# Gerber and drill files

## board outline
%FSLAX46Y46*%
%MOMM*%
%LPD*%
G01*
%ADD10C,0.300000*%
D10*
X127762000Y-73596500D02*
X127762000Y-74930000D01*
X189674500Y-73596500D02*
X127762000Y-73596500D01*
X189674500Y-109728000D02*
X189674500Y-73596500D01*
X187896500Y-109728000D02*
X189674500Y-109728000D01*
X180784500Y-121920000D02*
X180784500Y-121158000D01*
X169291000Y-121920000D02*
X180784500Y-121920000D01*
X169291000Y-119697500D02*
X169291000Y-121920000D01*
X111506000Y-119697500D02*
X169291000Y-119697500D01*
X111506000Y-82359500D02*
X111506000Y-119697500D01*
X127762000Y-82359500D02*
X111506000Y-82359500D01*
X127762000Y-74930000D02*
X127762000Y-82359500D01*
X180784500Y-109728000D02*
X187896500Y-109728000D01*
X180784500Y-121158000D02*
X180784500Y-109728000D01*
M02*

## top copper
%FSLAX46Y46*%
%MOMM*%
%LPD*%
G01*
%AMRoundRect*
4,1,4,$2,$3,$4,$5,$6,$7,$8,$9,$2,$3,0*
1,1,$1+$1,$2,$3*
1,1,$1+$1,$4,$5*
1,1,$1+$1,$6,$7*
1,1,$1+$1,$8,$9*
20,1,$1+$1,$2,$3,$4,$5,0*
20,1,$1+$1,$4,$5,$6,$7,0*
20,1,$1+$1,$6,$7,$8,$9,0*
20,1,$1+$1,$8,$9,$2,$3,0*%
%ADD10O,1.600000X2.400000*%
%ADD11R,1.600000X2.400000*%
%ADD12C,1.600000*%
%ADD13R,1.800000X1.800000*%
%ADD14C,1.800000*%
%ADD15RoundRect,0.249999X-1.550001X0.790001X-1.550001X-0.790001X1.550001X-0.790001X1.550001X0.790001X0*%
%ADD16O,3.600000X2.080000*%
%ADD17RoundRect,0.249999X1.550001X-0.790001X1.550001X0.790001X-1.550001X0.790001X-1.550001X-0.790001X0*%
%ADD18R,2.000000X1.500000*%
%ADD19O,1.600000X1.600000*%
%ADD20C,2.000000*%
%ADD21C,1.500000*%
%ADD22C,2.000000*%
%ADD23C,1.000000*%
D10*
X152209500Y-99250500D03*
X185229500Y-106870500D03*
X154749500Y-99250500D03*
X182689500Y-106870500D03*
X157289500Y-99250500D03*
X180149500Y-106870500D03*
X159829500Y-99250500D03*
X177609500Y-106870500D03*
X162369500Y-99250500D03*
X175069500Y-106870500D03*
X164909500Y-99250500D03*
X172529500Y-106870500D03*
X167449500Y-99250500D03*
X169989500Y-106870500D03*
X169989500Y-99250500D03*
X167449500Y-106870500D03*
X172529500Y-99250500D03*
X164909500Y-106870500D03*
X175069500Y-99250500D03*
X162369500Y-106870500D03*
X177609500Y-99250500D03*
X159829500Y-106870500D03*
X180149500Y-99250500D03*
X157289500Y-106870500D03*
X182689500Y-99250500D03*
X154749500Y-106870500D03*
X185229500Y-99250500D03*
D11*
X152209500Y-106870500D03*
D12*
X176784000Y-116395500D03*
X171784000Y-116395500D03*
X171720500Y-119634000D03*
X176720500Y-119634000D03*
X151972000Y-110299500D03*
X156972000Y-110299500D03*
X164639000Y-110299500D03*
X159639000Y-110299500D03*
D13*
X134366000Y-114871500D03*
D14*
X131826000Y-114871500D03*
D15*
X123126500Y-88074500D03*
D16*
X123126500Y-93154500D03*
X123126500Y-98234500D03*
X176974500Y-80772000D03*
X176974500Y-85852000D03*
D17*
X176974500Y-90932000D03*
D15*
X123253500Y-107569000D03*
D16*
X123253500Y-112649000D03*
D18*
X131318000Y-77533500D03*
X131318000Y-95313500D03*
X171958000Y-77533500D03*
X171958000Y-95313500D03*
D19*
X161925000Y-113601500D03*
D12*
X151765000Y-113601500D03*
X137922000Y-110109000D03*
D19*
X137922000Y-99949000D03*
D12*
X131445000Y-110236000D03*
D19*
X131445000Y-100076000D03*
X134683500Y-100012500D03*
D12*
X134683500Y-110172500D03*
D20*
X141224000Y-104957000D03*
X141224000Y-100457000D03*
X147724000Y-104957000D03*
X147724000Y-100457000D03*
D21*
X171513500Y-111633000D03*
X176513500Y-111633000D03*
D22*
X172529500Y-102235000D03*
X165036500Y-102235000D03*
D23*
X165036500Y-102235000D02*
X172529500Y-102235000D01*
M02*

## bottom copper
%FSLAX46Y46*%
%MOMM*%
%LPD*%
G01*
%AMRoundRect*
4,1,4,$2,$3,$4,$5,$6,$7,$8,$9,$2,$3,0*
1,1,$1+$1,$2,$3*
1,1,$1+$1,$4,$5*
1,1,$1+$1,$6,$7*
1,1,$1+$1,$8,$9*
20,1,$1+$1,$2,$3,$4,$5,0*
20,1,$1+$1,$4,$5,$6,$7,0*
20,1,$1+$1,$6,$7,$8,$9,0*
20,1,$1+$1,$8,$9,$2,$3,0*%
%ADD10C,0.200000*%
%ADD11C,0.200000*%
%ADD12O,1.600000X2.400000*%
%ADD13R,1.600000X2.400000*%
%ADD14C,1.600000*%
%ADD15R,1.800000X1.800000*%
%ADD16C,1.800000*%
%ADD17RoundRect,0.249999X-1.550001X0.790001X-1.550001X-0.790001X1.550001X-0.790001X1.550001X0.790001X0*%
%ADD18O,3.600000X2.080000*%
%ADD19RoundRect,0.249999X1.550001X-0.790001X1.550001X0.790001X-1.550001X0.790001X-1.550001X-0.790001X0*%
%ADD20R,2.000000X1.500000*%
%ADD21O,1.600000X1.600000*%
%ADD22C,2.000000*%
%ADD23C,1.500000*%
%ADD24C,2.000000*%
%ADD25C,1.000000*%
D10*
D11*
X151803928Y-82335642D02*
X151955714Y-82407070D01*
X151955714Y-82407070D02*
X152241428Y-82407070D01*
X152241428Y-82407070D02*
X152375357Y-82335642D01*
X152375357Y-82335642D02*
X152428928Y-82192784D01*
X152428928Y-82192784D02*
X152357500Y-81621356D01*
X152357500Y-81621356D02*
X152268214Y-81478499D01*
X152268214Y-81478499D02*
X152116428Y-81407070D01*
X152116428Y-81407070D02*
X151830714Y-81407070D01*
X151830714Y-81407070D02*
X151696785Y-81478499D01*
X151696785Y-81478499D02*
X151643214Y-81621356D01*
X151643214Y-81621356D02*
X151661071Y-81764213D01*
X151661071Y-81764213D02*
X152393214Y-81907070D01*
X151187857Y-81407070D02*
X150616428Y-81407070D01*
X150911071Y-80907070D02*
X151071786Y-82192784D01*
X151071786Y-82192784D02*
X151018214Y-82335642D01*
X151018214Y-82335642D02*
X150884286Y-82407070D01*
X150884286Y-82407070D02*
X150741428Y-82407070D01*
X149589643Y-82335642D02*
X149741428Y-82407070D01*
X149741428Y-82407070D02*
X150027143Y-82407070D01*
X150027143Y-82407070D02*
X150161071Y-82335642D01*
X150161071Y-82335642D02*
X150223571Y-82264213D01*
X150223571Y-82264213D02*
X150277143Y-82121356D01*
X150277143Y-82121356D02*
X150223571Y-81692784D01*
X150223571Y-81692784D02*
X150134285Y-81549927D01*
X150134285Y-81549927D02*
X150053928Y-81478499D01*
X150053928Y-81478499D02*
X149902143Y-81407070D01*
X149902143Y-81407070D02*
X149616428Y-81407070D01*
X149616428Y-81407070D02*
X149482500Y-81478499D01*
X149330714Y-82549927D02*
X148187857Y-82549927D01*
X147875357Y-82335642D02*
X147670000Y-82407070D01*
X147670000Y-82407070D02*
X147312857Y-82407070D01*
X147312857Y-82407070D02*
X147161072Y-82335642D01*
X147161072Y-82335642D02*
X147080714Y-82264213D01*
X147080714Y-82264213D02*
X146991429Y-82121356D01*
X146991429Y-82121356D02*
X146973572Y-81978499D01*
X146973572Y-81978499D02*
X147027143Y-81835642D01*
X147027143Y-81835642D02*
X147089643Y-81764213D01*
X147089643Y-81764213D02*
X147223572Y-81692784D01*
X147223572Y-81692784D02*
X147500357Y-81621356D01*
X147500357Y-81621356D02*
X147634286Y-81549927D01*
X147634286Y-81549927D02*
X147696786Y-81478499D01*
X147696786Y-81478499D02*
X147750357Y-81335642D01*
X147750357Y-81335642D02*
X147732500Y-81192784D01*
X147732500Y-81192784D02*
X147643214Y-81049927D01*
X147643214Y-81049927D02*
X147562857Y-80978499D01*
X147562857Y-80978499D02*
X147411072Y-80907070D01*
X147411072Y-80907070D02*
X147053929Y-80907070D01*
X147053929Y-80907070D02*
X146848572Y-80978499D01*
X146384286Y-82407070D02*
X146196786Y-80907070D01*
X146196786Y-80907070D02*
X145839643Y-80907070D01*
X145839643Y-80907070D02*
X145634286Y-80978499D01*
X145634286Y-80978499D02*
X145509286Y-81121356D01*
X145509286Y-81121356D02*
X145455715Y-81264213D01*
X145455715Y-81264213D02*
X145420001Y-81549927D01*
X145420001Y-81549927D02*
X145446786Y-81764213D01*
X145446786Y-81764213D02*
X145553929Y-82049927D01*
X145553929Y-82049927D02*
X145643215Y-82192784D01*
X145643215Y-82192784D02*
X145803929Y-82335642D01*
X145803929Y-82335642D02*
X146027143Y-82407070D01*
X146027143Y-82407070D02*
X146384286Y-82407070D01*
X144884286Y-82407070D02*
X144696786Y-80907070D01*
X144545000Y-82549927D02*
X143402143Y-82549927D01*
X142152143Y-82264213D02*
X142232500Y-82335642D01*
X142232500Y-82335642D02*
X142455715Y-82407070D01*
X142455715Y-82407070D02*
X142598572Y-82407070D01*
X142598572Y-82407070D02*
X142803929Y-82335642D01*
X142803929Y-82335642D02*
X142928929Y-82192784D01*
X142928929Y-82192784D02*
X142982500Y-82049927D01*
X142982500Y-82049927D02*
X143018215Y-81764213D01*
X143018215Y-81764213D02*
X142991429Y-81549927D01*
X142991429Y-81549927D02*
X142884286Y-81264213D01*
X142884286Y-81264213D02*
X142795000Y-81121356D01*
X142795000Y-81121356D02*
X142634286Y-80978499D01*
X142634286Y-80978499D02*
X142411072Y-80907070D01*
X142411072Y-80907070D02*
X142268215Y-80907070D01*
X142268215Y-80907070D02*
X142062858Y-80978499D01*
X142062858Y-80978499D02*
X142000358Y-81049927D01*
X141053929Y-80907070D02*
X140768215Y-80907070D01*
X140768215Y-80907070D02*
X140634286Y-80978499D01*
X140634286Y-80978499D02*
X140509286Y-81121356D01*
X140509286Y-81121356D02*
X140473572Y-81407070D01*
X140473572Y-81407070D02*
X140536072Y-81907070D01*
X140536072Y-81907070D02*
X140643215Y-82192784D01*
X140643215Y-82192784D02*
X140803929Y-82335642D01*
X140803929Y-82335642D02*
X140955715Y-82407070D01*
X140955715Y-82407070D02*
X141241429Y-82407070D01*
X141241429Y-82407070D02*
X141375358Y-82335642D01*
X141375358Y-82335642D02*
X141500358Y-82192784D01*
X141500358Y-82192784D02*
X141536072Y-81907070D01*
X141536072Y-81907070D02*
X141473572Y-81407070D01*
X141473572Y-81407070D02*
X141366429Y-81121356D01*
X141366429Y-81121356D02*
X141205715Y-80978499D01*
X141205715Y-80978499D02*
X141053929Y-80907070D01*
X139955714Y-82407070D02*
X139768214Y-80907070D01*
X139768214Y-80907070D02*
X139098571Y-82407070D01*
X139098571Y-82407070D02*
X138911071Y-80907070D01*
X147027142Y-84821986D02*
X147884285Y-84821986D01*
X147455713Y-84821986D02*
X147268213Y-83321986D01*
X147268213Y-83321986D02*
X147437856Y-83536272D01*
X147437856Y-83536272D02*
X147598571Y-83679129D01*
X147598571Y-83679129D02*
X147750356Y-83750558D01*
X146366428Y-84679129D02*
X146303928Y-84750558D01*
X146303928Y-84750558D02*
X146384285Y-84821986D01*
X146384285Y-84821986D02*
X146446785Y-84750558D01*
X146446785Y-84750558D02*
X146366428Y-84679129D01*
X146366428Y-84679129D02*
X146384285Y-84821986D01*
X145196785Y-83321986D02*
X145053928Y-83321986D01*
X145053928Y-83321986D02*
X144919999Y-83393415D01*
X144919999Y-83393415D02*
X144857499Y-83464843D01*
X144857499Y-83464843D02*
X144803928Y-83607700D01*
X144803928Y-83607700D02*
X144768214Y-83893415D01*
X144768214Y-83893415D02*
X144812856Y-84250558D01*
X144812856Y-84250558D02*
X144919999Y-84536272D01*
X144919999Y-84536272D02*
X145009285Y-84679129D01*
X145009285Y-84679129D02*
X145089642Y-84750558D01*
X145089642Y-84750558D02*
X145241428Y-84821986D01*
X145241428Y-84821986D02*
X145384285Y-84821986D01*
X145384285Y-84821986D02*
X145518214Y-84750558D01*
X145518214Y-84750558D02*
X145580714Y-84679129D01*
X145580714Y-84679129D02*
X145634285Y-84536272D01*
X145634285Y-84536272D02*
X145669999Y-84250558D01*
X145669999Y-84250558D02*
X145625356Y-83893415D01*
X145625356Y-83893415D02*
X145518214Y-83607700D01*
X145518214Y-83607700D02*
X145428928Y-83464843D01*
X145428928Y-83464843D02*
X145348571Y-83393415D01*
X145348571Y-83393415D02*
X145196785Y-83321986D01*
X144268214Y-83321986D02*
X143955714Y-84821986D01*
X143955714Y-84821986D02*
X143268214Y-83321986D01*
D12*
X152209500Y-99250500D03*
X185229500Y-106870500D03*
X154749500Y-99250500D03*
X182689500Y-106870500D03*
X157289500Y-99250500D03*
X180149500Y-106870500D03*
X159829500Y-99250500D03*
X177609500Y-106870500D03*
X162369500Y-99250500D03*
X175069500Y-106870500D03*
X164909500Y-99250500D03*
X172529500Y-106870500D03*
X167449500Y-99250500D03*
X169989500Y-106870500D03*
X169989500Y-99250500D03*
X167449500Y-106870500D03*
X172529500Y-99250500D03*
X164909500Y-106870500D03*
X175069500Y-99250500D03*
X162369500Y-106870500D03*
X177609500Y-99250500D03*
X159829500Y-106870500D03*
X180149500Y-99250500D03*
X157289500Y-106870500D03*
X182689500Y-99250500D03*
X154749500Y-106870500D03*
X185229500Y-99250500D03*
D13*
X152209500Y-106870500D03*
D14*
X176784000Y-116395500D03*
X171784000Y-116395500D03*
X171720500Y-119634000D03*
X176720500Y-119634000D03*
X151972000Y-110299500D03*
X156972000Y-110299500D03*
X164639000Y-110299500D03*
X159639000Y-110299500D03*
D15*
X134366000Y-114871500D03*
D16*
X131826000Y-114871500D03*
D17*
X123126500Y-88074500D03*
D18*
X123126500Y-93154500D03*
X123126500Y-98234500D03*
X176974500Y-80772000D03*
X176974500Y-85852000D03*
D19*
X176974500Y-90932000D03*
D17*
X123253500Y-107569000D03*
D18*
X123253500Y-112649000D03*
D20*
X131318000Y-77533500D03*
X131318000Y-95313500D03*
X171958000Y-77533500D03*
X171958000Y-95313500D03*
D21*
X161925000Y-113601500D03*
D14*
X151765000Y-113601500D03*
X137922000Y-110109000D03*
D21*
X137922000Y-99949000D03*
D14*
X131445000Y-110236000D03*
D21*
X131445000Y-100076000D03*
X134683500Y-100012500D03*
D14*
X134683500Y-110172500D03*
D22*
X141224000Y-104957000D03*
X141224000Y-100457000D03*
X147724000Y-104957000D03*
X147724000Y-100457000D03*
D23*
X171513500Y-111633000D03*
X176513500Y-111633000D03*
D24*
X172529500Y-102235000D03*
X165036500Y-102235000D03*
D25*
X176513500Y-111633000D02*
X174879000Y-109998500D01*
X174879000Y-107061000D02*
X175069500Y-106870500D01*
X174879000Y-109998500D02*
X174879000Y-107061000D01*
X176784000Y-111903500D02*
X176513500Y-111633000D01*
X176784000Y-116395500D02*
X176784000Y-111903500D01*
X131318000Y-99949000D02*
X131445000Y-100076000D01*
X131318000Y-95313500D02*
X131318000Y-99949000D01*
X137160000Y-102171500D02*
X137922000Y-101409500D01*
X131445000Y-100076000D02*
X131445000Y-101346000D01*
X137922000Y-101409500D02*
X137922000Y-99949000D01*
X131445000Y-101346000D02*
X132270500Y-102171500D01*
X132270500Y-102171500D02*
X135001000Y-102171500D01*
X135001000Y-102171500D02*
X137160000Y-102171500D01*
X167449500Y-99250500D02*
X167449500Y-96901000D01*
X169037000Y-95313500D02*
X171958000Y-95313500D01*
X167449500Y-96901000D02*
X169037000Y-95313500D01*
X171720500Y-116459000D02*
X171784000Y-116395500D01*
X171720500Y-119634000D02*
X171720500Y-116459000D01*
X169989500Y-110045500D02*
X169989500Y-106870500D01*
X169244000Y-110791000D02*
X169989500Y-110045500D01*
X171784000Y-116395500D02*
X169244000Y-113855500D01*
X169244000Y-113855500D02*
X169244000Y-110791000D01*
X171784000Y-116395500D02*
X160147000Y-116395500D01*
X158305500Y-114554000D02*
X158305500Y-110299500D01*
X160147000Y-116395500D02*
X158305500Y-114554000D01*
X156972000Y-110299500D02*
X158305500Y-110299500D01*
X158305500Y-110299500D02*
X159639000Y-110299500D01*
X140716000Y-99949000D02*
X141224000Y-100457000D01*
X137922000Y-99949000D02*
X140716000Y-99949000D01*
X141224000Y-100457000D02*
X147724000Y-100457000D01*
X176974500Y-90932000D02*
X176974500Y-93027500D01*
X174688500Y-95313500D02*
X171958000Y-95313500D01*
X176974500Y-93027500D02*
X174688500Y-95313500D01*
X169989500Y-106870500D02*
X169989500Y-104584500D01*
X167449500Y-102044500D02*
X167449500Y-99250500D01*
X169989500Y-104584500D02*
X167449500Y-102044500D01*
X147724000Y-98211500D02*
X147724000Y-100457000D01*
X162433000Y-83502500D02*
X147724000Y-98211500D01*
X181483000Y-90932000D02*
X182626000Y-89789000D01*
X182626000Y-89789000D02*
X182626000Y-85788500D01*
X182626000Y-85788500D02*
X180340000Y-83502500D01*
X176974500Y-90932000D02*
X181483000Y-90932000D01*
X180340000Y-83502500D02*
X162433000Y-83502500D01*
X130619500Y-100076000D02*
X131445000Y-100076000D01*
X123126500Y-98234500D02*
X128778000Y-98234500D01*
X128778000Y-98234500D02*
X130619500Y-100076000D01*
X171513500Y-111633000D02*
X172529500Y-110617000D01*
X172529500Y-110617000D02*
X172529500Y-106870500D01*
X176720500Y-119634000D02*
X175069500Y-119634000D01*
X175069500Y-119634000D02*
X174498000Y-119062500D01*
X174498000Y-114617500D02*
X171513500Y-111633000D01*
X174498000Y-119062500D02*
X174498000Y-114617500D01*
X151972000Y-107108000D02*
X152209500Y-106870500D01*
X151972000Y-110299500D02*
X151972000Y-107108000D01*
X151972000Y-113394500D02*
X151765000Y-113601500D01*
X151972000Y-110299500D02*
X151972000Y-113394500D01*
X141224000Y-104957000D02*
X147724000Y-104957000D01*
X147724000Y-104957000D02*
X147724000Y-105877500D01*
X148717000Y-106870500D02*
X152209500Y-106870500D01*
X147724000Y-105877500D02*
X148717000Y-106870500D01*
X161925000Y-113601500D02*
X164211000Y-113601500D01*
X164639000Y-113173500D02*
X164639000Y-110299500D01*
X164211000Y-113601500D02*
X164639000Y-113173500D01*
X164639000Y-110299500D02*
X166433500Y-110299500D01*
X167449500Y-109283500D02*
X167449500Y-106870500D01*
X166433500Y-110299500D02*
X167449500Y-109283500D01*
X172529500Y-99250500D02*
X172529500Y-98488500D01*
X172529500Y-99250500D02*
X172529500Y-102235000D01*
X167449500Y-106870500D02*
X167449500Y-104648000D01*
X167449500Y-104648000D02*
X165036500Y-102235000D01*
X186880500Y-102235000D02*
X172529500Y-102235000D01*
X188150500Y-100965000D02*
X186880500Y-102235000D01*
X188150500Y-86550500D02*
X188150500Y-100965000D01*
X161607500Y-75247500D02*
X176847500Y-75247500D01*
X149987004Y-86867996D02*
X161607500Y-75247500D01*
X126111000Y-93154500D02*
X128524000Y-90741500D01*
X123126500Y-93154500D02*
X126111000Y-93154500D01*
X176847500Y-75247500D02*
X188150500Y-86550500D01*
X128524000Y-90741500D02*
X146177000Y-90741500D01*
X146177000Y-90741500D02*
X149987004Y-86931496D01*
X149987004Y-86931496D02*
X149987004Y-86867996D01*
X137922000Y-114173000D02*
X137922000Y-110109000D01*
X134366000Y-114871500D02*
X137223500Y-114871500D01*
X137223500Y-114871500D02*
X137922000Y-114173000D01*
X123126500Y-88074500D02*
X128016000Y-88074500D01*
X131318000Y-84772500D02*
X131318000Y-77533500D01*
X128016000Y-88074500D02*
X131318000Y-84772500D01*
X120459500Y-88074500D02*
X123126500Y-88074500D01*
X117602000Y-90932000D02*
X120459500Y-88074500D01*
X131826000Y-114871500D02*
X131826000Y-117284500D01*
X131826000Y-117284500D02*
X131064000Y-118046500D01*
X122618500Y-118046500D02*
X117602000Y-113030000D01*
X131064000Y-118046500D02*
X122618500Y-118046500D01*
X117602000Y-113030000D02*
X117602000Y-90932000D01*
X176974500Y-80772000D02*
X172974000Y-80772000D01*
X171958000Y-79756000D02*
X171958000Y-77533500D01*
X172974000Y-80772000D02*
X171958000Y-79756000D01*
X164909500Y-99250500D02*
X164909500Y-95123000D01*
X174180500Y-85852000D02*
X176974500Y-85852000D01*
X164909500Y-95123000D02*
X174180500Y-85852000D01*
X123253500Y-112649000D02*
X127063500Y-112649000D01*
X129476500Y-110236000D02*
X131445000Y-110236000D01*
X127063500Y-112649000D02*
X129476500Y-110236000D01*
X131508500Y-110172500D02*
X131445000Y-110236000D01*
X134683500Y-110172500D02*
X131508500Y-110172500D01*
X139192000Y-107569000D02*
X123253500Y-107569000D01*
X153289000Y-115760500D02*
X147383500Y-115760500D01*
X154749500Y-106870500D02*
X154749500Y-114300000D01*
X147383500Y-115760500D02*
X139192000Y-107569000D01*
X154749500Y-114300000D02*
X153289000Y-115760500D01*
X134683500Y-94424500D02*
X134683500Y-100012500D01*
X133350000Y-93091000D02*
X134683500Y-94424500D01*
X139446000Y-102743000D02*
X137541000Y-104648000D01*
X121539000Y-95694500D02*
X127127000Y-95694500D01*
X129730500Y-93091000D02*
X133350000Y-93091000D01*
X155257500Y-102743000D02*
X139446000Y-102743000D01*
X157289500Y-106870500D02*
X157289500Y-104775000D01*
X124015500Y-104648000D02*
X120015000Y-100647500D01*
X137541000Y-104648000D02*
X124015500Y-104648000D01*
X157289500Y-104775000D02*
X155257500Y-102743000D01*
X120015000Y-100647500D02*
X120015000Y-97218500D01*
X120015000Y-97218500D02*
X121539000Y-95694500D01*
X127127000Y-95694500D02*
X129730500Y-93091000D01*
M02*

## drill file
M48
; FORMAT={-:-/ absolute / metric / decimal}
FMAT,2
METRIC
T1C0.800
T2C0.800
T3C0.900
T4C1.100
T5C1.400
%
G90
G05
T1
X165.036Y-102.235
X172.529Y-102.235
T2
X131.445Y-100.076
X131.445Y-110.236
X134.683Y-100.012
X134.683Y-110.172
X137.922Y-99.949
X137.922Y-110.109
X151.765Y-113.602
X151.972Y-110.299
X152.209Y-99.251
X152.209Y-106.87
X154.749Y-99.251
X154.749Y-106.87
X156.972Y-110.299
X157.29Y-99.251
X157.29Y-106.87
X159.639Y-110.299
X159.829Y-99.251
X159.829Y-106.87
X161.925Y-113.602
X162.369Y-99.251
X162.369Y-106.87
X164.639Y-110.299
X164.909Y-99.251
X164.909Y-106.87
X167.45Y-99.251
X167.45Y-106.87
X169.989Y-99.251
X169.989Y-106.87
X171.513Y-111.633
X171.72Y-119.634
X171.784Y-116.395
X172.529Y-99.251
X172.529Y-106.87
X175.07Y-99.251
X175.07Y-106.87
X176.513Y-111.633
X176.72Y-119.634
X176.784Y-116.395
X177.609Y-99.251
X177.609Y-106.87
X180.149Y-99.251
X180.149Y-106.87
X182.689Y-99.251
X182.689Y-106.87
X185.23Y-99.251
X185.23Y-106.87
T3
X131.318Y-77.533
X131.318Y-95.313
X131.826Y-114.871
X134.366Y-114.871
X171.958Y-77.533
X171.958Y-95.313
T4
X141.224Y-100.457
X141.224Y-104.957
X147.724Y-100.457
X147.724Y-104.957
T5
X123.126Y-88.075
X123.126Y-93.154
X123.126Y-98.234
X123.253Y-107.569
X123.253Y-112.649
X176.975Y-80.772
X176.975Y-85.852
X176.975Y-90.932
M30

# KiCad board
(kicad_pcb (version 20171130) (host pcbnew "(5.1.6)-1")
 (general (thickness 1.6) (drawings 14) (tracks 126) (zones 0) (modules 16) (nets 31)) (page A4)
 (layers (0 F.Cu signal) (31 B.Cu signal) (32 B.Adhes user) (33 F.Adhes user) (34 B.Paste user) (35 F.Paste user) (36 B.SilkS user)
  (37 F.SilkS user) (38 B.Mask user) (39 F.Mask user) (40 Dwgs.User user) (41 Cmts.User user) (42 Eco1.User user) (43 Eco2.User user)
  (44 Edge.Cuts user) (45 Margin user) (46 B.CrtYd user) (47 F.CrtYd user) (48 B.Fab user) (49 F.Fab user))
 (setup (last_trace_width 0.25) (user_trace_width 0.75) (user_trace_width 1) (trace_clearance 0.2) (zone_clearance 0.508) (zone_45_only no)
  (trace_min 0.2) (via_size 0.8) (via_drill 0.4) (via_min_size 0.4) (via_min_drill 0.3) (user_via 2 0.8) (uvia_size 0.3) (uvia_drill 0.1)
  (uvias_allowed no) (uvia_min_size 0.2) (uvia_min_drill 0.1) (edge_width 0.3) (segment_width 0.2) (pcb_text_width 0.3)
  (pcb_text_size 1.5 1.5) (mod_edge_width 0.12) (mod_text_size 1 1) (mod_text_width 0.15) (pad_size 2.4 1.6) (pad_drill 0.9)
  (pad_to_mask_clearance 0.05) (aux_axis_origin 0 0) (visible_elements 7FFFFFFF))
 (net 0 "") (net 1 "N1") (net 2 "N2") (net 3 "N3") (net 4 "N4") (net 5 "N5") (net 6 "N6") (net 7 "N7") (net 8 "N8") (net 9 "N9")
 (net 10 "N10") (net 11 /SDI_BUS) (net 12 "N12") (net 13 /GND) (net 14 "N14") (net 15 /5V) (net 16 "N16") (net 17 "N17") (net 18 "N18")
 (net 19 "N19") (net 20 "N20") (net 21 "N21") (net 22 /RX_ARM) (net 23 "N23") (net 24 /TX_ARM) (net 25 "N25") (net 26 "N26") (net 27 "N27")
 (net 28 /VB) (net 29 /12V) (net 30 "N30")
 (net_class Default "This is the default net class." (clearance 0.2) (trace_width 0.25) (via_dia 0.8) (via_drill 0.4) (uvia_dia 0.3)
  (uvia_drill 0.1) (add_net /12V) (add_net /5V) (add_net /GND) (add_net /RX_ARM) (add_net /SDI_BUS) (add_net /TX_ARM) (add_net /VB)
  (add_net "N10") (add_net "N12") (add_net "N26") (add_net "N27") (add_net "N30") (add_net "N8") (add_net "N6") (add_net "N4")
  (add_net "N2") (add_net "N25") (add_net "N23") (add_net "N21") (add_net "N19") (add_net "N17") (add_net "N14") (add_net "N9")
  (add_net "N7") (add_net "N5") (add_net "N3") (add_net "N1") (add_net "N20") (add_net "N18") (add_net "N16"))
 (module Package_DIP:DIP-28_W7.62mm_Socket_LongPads (layer F.Cu) (at 152.2095 106.8705 90)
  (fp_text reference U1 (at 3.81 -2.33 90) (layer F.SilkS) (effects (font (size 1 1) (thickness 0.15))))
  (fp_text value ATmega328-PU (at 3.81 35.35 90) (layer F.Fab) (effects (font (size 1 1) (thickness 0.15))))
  (pad 28 thru_hole oval (at 7.62 0 90) (size 2.4 1.6) (drill 0.8) (layers *.Cu *.Mask) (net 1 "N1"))
  (pad 14 thru_hole oval (at 0 33.02 90) (size 2.4 1.6) (drill 0.8) (layers *.Cu *.Mask) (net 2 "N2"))
  (pad 27 thru_hole oval (at 7.62 2.54 90) (size 2.4 1.6) (drill 0.8) (layers *.Cu *.Mask) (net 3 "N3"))
  (pad 13 thru_hole oval (at 0 30.48 90) (size 2.4 1.6) (drill 0.8) (layers *.Cu *.Mask) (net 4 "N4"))
  (pad 26 thru_hole oval (at 7.62 5.08 90) (size 2.4 1.6) (drill 0.8) (layers *.Cu *.Mask) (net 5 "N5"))
  (pad 12 thru_hole oval (at 0 27.94 90) (size 2.4 1.6) (drill 0.8) (layers *.Cu *.Mask) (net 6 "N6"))
  (pad 25 thru_hole oval (at 7.62 7.62 90) (size 2.4 1.6) (drill 0.8) (layers *.Cu *.Mask) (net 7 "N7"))
  (pad 11 thru_hole oval (at 0 25.4 90) (size 2.4 1.6) (drill 0.8) (layers *.Cu *.Mask) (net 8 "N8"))
  (pad 24 thru_hole oval (at 7.62 10.16 90) (size 2.4 1.6) (drill 0.8) (layers *.Cu *.Mask) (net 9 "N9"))
  (pad 10 thru_hole oval (at 0 22.86 90) (size 2.4 1.6) (drill 0.8) (layers *.Cu *.Mask) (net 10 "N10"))
  (pad 23 thru_hole oval (at 7.62 12.7 90) (size 2.4 1.6) (drill 0.8) (layers *.Cu *.Mask) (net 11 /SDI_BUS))
  (pad 9 thru_hole oval (at 0 20.32 90) (size 2.4 1.6) (drill 0.8) (layers *.Cu *.Mask) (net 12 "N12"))
  (pad 22 thru_hole oval (at 7.62 15.24 90) (size 2.4 1.6) (drill 0.8) (layers *.Cu *.Mask) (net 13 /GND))
  (pad 8 thru_hole oval (at 0 17.78 90) (size 2.4 1.6) (drill 0.8) (layers *.Cu *.Mask) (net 13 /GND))
  (pad 21 thru_hole oval (at 7.62 17.78 90) (size 2.4 1.6) (drill 0.8) (layers *.Cu *.Mask) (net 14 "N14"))
  (pad 7 thru_hole oval (at 0 15.24 90) (size 2.4 1.6) (drill 0.8) (layers *.Cu *.Mask) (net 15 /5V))
  (pad 20 thru_hole oval (at 7.62 20.32 90) (size 2.4 1.6) (drill 0.8) (layers *.Cu *.Mask) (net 15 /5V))
  (pad 6 thru_hole oval (at 0 12.7 90) (size 2.4 1.6) (drill 0.8) (layers *.Cu *.Mask) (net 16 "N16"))
  (pad 19 thru_hole oval (at 7.62 22.86 90) (size 2.4 1.6) (drill 0.8) (layers *.Cu *.Mask) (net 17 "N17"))
  (pad 5 thru_hole oval (at 0 10.16 90) (size 2.4 1.6) (drill 0.8) (layers *.Cu *.Mask) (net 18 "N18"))
  (pad 18 thru_hole oval (at 7.62 25.4 90) (size 2.4 1.6) (drill 0.8) (layers *.Cu *.Mask) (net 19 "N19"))
  (pad 4 thru_hole oval (at 0 7.62 90) (size 2.4 1.6) (drill 0.8) (layers *.Cu *.Mask) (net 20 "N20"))
  (pad 17 thru_hole oval (at 7.62 27.94 90) (size 2.4 1.6) (drill 0.8) (layers *.Cu *.Mask) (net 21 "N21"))
  (pad 3 thru_hole oval (at 0 5.08 90) (size 2.4 1.6) (drill 0.8) (layers *.Cu *.Mask) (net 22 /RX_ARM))
  (pad 16 thru_hole oval (at 7.62 30.48 90) (size 2.4 1.6) (drill 0.8) (layers *.Cu *.Mask) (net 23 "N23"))
  (pad 2 thru_hole oval (at 0 2.54 90) (size 2.4 1.6) (drill 0.8) (layers *.Cu *.Mask) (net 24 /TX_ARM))
  (pad 15 thru_hole oval (at 7.62 33.02 90) (size 2.4 1.6) (drill 0.8) (layers *.Cu *.Mask) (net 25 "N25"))
  (pad 1 thru_hole rect (at 0 0 90) (size 2.4 1.6) (drill 0.8) (layers *.Cu *.Mask) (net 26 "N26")))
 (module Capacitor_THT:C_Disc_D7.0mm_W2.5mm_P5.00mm (layer F.Cu) (at 176.784 116.3955 180)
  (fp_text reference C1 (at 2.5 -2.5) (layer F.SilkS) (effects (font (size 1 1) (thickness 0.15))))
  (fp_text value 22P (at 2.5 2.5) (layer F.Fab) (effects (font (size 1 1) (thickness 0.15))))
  (pad 1 thru_hole circle (at 0 0 180) (size 1.6 1.6) (drill 0.8) (layers *.Cu *.Mask) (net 10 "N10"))
  (pad 2 thru_hole circle (at 5 0 180) (size 1.6 1.6) (drill 0.8) (layers *.Cu *.Mask) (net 13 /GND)))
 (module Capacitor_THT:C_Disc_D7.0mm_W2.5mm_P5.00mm (layer F.Cu) (at 176.7205 119.634 180)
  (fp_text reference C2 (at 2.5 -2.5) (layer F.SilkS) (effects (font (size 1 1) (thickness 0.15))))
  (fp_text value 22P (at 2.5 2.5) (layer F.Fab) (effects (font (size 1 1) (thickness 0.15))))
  (pad 2 thru_hole circle (at 5 0 180) (size 1.6 1.6) (drill 0.8) (layers *.Cu *.Mask) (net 13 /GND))
  (pad 1 thru_hole circle (at 0 0 180) (size 1.6 1.6) (drill 0.8) (layers *.Cu *.Mask) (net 12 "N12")))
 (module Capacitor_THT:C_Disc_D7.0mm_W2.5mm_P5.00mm (layer F.Cu) (at 156.972 110.2995 180)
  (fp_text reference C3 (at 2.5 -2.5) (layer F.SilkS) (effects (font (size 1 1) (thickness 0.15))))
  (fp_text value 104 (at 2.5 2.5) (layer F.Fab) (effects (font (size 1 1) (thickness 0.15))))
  (pad 2 thru_hole circle (at 5 0 180) (size 1.6 1.6) (drill 0.8) (layers *.Cu *.Mask) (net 26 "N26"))
  (pad 1 thru_hole circle (at 0 0 180) (size 1.6 1.6) (drill 0.8) (layers *.Cu *.Mask) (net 13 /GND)))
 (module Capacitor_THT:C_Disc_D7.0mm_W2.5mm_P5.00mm (layer F.Cu) (at 164.639 110.2995 180)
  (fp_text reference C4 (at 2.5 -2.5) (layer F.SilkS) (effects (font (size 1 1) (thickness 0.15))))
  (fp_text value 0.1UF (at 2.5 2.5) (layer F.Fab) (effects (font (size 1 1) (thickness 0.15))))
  (pad 1 thru_hole circle (at 0 0 180) (size 1.6 1.6) (drill 0.8) (layers *.Cu *.Mask) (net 15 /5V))
  (pad 2 thru_hole circle (at 5 0 180) (size 1.6 1.6) (drill 0.8) (layers *.Cu *.Mask) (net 13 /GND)))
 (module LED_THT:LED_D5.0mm (layer F.Cu) (at 134.366 114.8715 180)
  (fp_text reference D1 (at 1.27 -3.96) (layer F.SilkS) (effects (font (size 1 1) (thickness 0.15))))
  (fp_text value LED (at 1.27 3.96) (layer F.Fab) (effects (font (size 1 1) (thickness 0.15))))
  (pad 1 thru_hole rect (at 0 0 180) (size 1.8 1.8) (drill 0.9) (layers *.Cu *.Mask) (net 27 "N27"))
  (pad 2 thru_hole circle (at 2.54 0 180) (size 1.8 1.8) (drill 0.9) (layers *.Cu *.Mask) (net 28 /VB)))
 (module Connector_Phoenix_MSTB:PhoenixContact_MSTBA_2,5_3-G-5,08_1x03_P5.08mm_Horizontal (layer F.Cu) (at 123.1265 88.0745 270)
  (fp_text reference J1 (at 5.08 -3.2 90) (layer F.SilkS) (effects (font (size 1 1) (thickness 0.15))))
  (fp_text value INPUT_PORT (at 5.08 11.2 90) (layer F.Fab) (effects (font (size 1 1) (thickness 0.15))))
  (pad 1 thru_hole roundrect (at 0 0 270) (size 2.08 3.6) (drill 1.4) (layers *.Cu *.Mask) (roundrect_rratio 0.120192) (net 28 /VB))
  (pad 2 thru_hole oval (at 5.08 0 270) (size 2.08 3.6) (drill 1.4) (layers *.Cu *.Mask) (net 15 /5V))
  (pad 3 thru_hole oval (at 10.16 0 270) (size 2.08 3.6) (drill 1.4) (layers *.Cu *.Mask) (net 13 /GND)))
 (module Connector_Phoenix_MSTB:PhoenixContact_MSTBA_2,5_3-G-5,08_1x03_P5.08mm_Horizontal (layer F.Cu) (at 176.9745 90.932 90)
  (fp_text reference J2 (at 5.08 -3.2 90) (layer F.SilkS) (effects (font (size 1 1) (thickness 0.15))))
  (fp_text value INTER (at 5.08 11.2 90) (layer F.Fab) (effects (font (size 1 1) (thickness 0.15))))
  (pad 3 thru_hole oval (at 10.16 0 90) (size 2.08 3.6) (drill 1.4) (layers *.Cu *.Mask) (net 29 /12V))
  (pad 2 thru_hole oval (at 5.08 0 90) (size 2.08 3.6) (drill 1.4) (layers *.Cu *.Mask) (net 11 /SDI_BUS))
  (pad 1 thru_hole roundrect (at 0 0 90) (size 2.08 3.6) (drill 1.4) (layers *.Cu *.Mask) (roundrect_rratio 0.120192) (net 13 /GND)))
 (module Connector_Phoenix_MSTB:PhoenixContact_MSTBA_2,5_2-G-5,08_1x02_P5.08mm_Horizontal (layer F.Cu) (at 123.2535 107.569 270)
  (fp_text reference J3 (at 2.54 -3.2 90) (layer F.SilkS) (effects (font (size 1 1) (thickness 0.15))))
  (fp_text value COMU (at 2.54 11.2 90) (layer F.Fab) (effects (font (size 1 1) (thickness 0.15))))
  (pad 1 thru_hole roundrect (at 0 0 270) (size 2.08 3.6) (drill 1.4) (layers *.Cu *.Mask) (roundrect_rratio 0.120192) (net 24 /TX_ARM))
  (pad 2 thru_hole oval (at 5.08 0 270) (size 2.08 3.6) (drill 1.4) (layers *.Cu *.Mask) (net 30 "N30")))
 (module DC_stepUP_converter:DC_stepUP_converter (layer F.Cu) (at 151.638 71.1835)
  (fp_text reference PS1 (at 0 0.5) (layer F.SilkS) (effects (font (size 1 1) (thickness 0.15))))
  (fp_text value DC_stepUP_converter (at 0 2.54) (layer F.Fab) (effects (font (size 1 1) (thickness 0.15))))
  (pad 1 thru_hole rect (at -20.32 6.35) (size 2 1.5) (drill 0.9) (layers *.Cu *.Mask) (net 28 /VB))
  (pad 2 thru_hole rect (at -20.32 24.13) (size 2 1.5) (drill 0.9) (layers *.Cu *.Mask) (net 13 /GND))
  (pad 3 thru_hole rect (at 20.32 6.35) (size 2 1.5) (drill 0.9) (layers *.Cu *.Mask) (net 29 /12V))
  (pad 4 thru_hole rect (at 20.32 24.13) (size 2 1.5) (drill 0.9) (layers *.Cu *.Mask) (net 13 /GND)))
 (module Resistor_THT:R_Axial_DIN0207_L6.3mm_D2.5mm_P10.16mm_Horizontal (layer F.Cu) (at 151.765 113.6015)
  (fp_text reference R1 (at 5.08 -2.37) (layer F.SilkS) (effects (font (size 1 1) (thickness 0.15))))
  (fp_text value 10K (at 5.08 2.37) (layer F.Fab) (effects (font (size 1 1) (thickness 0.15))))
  (pad 2 thru_hole oval (at 10.16 0) (size 1.6 1.6) (drill 0.8) (layers *.Cu *.Mask) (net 15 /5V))
  (pad 1 thru_hole circle (at 0 0) (size 1.6 1.6) (drill 0.8) (layers *.Cu *.Mask) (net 26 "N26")))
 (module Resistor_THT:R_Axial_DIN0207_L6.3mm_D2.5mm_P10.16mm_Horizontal (layer F.Cu) (at 137.922 110.109 90)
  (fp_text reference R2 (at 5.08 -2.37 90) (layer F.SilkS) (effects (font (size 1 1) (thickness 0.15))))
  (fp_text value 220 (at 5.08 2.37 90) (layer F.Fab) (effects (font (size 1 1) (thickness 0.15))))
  (pad 1 thru_hole circle (at 0 0 90) (size 1.6 1.6) (drill 0.8) (layers *.Cu *.Mask) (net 27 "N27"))
  (pad 2 thru_hole oval (at 10.16 0 90) (size 1.6 1.6) (drill 0.8) (layers *.Cu *.Mask) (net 13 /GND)))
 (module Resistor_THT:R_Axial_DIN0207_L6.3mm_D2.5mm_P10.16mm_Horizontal (layer F.Cu) (at 131.445 110.236 90)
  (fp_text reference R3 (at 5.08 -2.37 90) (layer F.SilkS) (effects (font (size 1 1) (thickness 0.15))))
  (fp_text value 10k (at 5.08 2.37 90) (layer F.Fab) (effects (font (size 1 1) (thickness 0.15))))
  (pad 1 thru_hole circle (at 0 0 90) (size 1.6 1.6) (drill 0.8) (layers *.Cu *.Mask) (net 30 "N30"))
  (pad 2 thru_hole oval (at 10.16 0 90) (size 1.6 1.6) (drill 0.8) (layers *.Cu *.Mask) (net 13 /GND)))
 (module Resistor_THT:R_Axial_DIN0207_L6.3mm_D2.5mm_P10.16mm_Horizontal (layer F.Cu) (at 134.6835 110.1725 90)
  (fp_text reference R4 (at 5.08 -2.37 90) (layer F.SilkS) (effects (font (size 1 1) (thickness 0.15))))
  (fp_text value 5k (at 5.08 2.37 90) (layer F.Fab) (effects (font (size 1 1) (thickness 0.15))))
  (pad 2 thru_hole oval (at 10.16 0 90) (size 1.6 1.6) (drill 0.8) (layers *.Cu *.Mask) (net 22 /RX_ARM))
  (pad 1 thru_hole circle (at 0 0 90) (size 1.6 1.6) (drill 0.8) (layers *.Cu *.Mask) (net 30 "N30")))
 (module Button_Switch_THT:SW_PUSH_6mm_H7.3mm (layer F.Cu) (at 141.224 100.457)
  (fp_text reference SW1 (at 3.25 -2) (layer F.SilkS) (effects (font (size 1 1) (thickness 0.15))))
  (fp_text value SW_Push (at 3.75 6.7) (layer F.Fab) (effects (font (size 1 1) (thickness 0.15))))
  (pad 2 thru_hole circle (at 0 4.5 90) (size 2 2) (drill 1.1) (layers *.Cu *.Mask) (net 26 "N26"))
  (pad 1 thru_hole circle (at 0 0 90) (size 2 2) (drill 1.1) (layers *.Cu *.Mask) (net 13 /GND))
  (pad 2 thru_hole circle (at 6.5 4.5 90) (size 2 2) (drill 1.1) (layers *.Cu *.Mask) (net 26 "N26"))
  (pad 1 thru_hole circle (at 6.5 0 90) (size 2 2) (drill 1.1) (layers *.Cu *.Mask) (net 13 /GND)))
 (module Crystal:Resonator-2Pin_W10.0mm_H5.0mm (layer F.Cu) (at 171.5135 111.633)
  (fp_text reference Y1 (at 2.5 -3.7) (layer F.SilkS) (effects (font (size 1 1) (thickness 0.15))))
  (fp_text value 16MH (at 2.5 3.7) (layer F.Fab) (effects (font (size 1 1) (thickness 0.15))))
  (pad 1 thru_hole circle (at 0 0) (size 1.5 1.5) (drill 0.8) (layers *.Cu *.Mask) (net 12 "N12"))
  (pad 2 thru_hole circle (at 5 0) (size 1.5 1.5) (drill 0.8) (layers *.Cu *.Mask) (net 10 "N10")))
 (gr_line (start 127.762 73.5965) (end 127.762 74.93) (layer Edge.Cuts) (width 0.3))
 (gr_line (start 189.6745 73.5965) (end 127.762 73.5965) (layer Edge.Cuts) (width 0.3))
 (gr_line (start 189.6745 109.728) (end 189.6745 73.5965) (layer Edge.Cuts) (width 0.3))
 (gr_line (start 187.8965 109.728) (end 189.6745 109.728) (layer Edge.Cuts) (width 0.3))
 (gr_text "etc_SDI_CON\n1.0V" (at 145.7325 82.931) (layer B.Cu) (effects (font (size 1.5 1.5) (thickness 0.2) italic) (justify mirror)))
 (gr_line (start 180.7845 121.92) (end 180.7845 121.158) (layer Edge.Cuts) (width 0.3))
 (gr_line (start 169.291 121.92) (end 180.7845 121.92) (layer Edge.Cuts) (width 0.3))
 (gr_line (start 169.291 119.6975) (end 169.291 121.92) (layer Edge.Cuts) (width 0.3))
 (gr_line (start 111.506 119.6975) (end 169.291 119.6975) (layer Edge.Cuts) (width 0.3))
 (gr_line (start 111.506 82.3595) (end 111.506 119.6975) (layer Edge.Cuts) (width 0.3))
 (gr_line (start 127.762 82.3595) (end 111.506 82.3595) (layer Edge.Cuts) (width 0.3))
 (gr_line (start 127.762 74.93) (end 127.762 82.3595) (layer Edge.Cuts) (width 0.3))
 (gr_line (start 180.7845 109.728) (end 187.8965 109.728) (layer Edge.Cuts) (width 0.3))
 (gr_line (start 180.7845 121.158) (end 180.7845 109.728) (layer Edge.Cuts) (width 0.3))
 (segment (start 176.5135 111.633) (end 174.879 109.9985) (width 1) (layer B.Cu) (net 10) (status 10))
 (segment (start 174.879 107.061) (end 175.0695 106.8705) (width 1) (layer B.Cu) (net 10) (status 30))
 (segment (start 174.879 109.9985) (end 174.879 107.061) (width 1) (layer B.Cu) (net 10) (status 20))
 (segment (start 176.784 111.9035) (end 176.5135 111.633) (width 1) (layer B.Cu) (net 10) (status 30))
 (segment (start 176.784 116.3955) (end 176.784 111.9035) (width 1) (layer B.Cu) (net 10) (status 30))
 (segment (start 131.318 99.949) (end 131.445 100.076) (width 1) (layer B.Cu) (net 13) (status 30))
 (segment (start 131.318 95.3135) (end 131.318 99.949) (width 1) (layer B.Cu) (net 13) (status 30))
 (segment (start 137.16 102.1715) (end 137.922 101.4095) (width 1) (layer B.Cu) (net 13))
 (segment (start 131.445 100.076) (end 131.445 101.346) (width 1) (layer B.Cu) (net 13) (status 10))
 (segment (start 137.922 101.4095) (end 137.922 99.949) (width 1) (layer B.Cu) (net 13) (status 20))
 (segment (start 131.445 101.346) (end 132.2705 102.1715) (width 1) (layer B.Cu) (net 13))
 (segment (start 132.2705 102.1715) (end 135.001 102.1715) (width 1) (layer B.Cu) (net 13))
 (segment (start 135.001 102.1715) (end 137.16 102.1715) (width 1) (layer B.Cu) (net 13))
 (segment (start 167.4495 99.2505) (end 167.4495 96.901) (width 1) (layer B.Cu) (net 13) (status 10))
 (segment (start 169.037 95.3135) (end 171.958 95.3135) (width 1) (layer B.Cu) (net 13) (status 20))
 (segment (start 167.4495 96.901) (end 169.037 95.3135) (width 1) (layer B.Cu) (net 13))
 (segment (start 171.7205 116.459) (end 171.784 116.3955) (width 1) (layer B.Cu) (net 13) (status 30))
 (segment (start 171.7205 119.634) (end 171.7205 116.459) (width 1) (layer B.Cu) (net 13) (status 30))
 (segment (start 169.9895 110.0455) (end 169.9895 106.8705) (width 1) (layer B.Cu) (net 13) (status 20))
 (segment (start 169.244 110.791) (end 169.9895 110.0455) (width 1) (layer B.Cu) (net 13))
 (segment (start 171.784 116.3955) (end 169.244 113.8555) (width 1) (layer B.Cu) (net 13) (status 10))
 (segment (start 169.244 113.8555) (end 169.244 110.791) (width 1) (layer B.Cu) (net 13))
 (segment (start 171.784 116.3955) (end 160.147 116.3955) (width 1) (layer B.Cu) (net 13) (status 10))
 (segment (start 158.3055 114.554) (end 158.3055 110.2995) (width 1) (layer B.Cu) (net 13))
 (segment (start 160.147 116.3955) (end 158.3055 114.554) (width 1) (layer B.Cu) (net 13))
 (segment (start 156.972 110.2995) (end 158.3055 110.2995) (width 1) (layer B.Cu) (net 13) (status 10))
 (segment (start 158.3055 110.2995) (end 159.639 110.2995) (width 1) (layer B.Cu) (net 13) (status 20))
 (segment (start 140.716 99.949) (end 141.224 100.457) (width 1) (layer B.Cu) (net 13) (status 30))
 (segment (start 137.922 99.949) (end 140.716 99.949) (width 1) (layer B.Cu) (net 13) (status 30))
 (segment (start 141.224 100.457) (end 147.724 100.457) (width 1) (layer B.Cu) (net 13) (status 30))
 (segment (start 176.9745 90.932) (end 176.9745 93.0275) (width 1) (layer B.Cu) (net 13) (status 10))
 (segment (start 174.6885 95.3135) (end 171.958 95.3135) (width 1) (layer B.Cu) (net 13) (status 20))
 (segment (start 176.9745 93.0275) (end 174.6885 95.3135) (width 1) (layer B.Cu) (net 13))
 (segment (start 169.9895 106.8705) (end 169.9895 104.5845) (width 1) (layer B.Cu) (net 13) (status 10))
 (segment (start 167.4495 102.0445) (end 167.4495 99.2505) (width 1) (layer B.Cu) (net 13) (status 20))
 (segment (start 169.9895 104.5845) (end 167.4495 102.0445) (width 1) (layer B.Cu) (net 13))
 (segment (start 147.724 98.2115) (end 147.724 100.457) (width 1) (layer B.Cu) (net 13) (status 20))
 (segment (start 162.433 83.5025) (end 147.724 98.2115) (width 1) (layer B.Cu) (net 13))
 (segment (start 181.483 90.932) (end 182.626 89.789) (width 1) (layer B.Cu) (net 13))
 (segment (start 182.626 89.789) (end 182.626 85.7885) (width 1) (layer B.Cu) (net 13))
 (segment (start 182.626 85.7885) (end 180.34 83.5025) (width 1) (layer B.Cu) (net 13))
 (segment (start 176.9745 90.932) (end 181.483 90.932) (width 1) (layer B.Cu) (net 13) (status 10))
 (segment (start 180.34 83.5025) (end 162.433 83.5025) (width 1) (layer B.Cu) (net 13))
 (segment (start 130.6195 100.076) (end 131.445 100.076) (width 1) (layer B.Cu) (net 13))
 (segment (start 123.1265 98.2345) (end 128.778 98.2345) (width 1) (layer B.Cu) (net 13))
 (segment (start 128.778 98.2345) (end 130.6195 100.076) (width 1) (layer B.Cu) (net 13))
 (segment (start 171.5135 111.633) (end 172.5295 110.617) (width 1) (layer B.Cu) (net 12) (status 10))
 (segment (start 172.5295 110.617) (end 172.5295 106.8705) (width 1) (layer B.Cu) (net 12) (status 20))
 (segment (start 176.7205 119.634) (end 175.0695 119.634) (width 1) (layer B.Cu) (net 12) (status 10))
 (segment (start 175.0695 119.634) (end 174.498 119.0625) (width 1) (layer B.Cu) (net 12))
 (segment (start 174.498 114.6175) (end 171.5135 111.633) (width 1) (layer B.Cu) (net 12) (status 20))
 (segment (start 174.498 119.0625) (end 174.498 114.6175) (width 1) (layer B.Cu) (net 12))
 (segment (start 151.972 107.108) (end 152.2095 106.8705) (width 1) (layer B.Cu) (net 26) (status 30))
 (segment (start 151.972 110.2995) (end 151.972 107.108) (width 1) (layer B.Cu) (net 26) (status 30))
 (segment (start 151.972 113.3945) (end 151.765 113.6015) (width 1) (layer B.Cu) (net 26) (status 30))
 (segment (start 151.972 110.2995) (end 151.972 113.3945) (width 1) (layer B.Cu) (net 26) (status 30))
 (segment (start 141.224 104.957) (end 147.724 104.957) (width 1) (layer B.Cu) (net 26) (status 30))
 (segment (start 147.724 104.957) (end 147.724 105.8775) (width 1) (layer B.Cu) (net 26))
 (segment (start 148.717 106.8705) (end 152.2095 106.8705) (width 1) (layer B.Cu) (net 26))
 (segment (start 147.724 105.8775) (end 148.717 106.8705) (width 1) (layer B.Cu) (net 26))
 (segment (start 161.925 113.6015) (end 164.211 113.6015) (width 1) (layer B.Cu) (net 15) (status 10))
 (segment (start 164.639 113.1735) (end 164.639 110.2995) (width 1) (layer B.Cu) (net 15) (status 20))
 (segment (start 164.211 113.6015) (end 164.639 113.1735) (width 1) (layer B.Cu) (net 15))
 (segment (start 164.639 110.2995) (end 166.4335 110.2995) (width 1) (layer B.Cu) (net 15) (status 10))
 (segment (start 167.4495 109.2835) (end 167.4495 106.8705) (width 1) (layer B.Cu) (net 15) (status 20))
 (segment (start 166.4335 110.2995) (end 167.4495 109.2835) (width 1) (layer B.Cu) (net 15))
 (segment (start 172.5295 99.2505) (end 172.5295 98.4885) (width 1) (layer B.Cu) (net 15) (status 30))
 (segment (start 172.5295 99.2505) (end 172.5295 102.235) (width 1) (layer B.Cu) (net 15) (status 10))
 (via (at 172.5295 102.235) (size 2) (drill 0.8) (layers F.Cu B.Cu) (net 15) (status 1000000))
 (segment (start 167.4495 106.8705) (end 167.4495 104.648) (width 1) (layer B.Cu) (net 15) (status 10))
 (via (at 165.0365 102.235) (size 2) (drill 0.8) (layers F.Cu B.Cu) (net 15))
 (segment (start 167.4495 104.648) (end 165.0365 102.235) (width 1) (layer B.Cu) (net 15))
 (segment (start 165.0365 102.235) (end 172.5295 102.235) (width 1) (layer F.Cu) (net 15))
 (segment (start 186.8805 102.235) (end 172.5295 102.235) (width 1) (layer B.Cu) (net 15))
 (segment (start 188.1505 100.965) (end 186.8805 102.235) (width 1) (layer B.Cu) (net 15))
 (segment (start 188.1505 86.5505) (end 188.1505 100.965) (width 1) (layer B.Cu) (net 15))
 (segment (start 161.6075 75.2475) (end 176.8475 75.2475) (width 1) (layer B.Cu) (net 15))
 (segment (start 149.987004 86.867996) (end 161.6075 75.2475) (width 1) (layer B.Cu) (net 15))
 (segment (start 126.111 93.1545) (end 128.524 90.7415) (width 1) (layer B.Cu) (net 15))
 (segment (start 123.1265 93.1545) (end 126.111 93.1545) (width 1) (layer B.Cu) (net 15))
 (segment (start 176.8475 75.2475) (end 188.1505 86.5505) (width 1) (layer B.Cu) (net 15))
 (segment (start 128.524 90.7415) (end 146.177 90.7415) (width 1) (layer B.Cu) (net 15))
 (segment (start 146.177 90.7415) (end 149.987004 86.931496) (width 1) (layer B.Cu) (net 15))
 (segment (start 149.987004 86.931496) (end 149.987004 86.867996) (width 1) (layer B.Cu) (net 15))
 (segment (start 137.922 114.173) (end 137.922 110.109) (width 1) (layer B.Cu) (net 27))
 (segment (start 134.366 114.8715) (end 137.2235 114.8715) (width 1) (layer B.Cu) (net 27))
 (segment (start 137.2235 114.8715) (end 137.922 114.173) (width 1) (layer B.Cu) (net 27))
 (segment (start 123.1265 88.0745) (end 128.016 88.0745) (width 1) (layer B.Cu) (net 28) (status 10))
 (segment (start 131.318 84.7725) (end 131.318 77.5335) (width 1) (layer B.Cu) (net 28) (status 20))
 (segment (start 128.016 88.0745) (end 131.318 84.7725) (width 1) (layer B.Cu) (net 28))
 (segment (start 120.4595 88.0745) (end 123.1265 88.0745) (width 1) (layer B.Cu) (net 28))
 (segment (start 117.602 90.932) (end 120.4595 88.0745) (width 1) (layer B.Cu) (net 28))
 (segment (start 131.826 114.8715) (end 131.826 117.2845) (width 1) (layer B.Cu) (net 28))
 (segment (start 131.826 117.2845) (end 131.064 118.0465) (width 1) (layer B.Cu) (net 28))
 (segment (start 122.6185 118.0465) (end 117.602 113.03) (width 1) (layer B.Cu) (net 28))
 (segment (start 131.064 118.0465) (end 122.6185 118.0465) (width 1) (layer B.Cu) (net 28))
 (segment (start 117.602 113.03) (end 117.602 90.932) (width 1) (layer B.Cu) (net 28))
 (segment (start 176.9745 80.772) (end 172.974 80.772) (width 1) (layer B.Cu) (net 29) (status 10))
 (segment (start 171.958 79.756) (end 171.958 77.5335) (width 1) (layer B.Cu) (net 29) (status 20))
 (segment (start 172.974 80.772) (end 171.958 79.756) (width 1) (layer B.Cu) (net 29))
 (segment (start 164.9095 99.2505) (end 164.9095 95.123) (width 1) (layer B.Cu) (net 11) (status 10))
 (segment (start 174.1805 85.852) (end 176.9745 85.852) (width 1) (layer B.Cu) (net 11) (status 20))
 (segment (start 164.9095 95.123) (end 174.1805 85.852) (width 1) (layer B.Cu) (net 11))
 (segment (start 123.2535 112.649) (end 127.0635 112.649) (width 1) (layer B.Cu) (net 30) (status 10))
 (segment (start 129.4765 110.236) (end 131.445 110.236) (width 1) (layer B.Cu) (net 30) (status 20))
 (segment (start 127.0635 112.649) (end 129.4765 110.236) (width 1) (layer B.Cu) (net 30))
 (segment (start 131.5085 110.1725) (end 131.445 110.236) (width 1) (layer B.Cu) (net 30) (status 30))
 (segment (start 134.6835 110.1725) (end 131.5085 110.1725) (width 1) (layer B.Cu) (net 30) (status 30))
 (segment (start 139.192 107.569) (end 123.2535 107.569) (width 1) (layer B.Cu) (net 24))
 (segment (start 153.289 115.7605) (end 147.3835 115.7605) (width 1) (layer B.Cu) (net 24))
 (segment (start 154.7495 106.8705) (end 154.7495 114.3) (width 1) (layer B.Cu) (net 24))
 (segment (start 147.3835 115.7605) (end 139.192 107.569) (width 1) (layer B.Cu) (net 24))
 (segment (start 154.7495 114.3) (end 153.289 115.7605) (width 1) (layer B.Cu) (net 24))
 (segment (start 134.6835 94.4245) (end 134.6835 100.0125) (width 1) (layer B.Cu) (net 22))
 (segment (start 133.35 93.091) (end 134.6835 94.4245) (width 1) (layer B.Cu) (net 22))
 (segment (start 139.446 102.743) (end 137.541 104.648) (width 1) (layer B.Cu) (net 22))
 (segment (start 121.539 95.6945) (end 127.127 95.6945) (width 1) (layer B.Cu) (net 22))
 (segment (start 129.7305 93.091) (end 133.35 93.091) (width 1) (layer B.Cu) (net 22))
 (segment (start 155.2575 102.743) (end 139.446 102.743) (width 1) (layer B.Cu) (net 22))
 (segment (start 157.2895 106.8705) (end 157.2895 104.775) (width 1) (layer B.Cu) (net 22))
 (segment (start 124.0155 104.648) (end 120.015 100.6475) (width 1) (layer B.Cu) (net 22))
 (segment (start 137.541 104.648) (end 124.0155 104.648) (width 1) (layer B.Cu) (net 22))
 (segment (start 157.2895 104.775) (end 155.2575 102.743) (width 1) (layer B.Cu) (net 22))
 (segment (start 120.015 100.6475) (end 120.015 97.2185) (width 1) (layer B.Cu) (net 22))
 (segment (start 120.015 97.2185) (end 121.539 95.6945) (width 1) (layer B.Cu) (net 22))
 (segment (start 127.127 95.6945) (end 129.7305 93.091) (width 1) (layer B.Cu) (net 22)))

